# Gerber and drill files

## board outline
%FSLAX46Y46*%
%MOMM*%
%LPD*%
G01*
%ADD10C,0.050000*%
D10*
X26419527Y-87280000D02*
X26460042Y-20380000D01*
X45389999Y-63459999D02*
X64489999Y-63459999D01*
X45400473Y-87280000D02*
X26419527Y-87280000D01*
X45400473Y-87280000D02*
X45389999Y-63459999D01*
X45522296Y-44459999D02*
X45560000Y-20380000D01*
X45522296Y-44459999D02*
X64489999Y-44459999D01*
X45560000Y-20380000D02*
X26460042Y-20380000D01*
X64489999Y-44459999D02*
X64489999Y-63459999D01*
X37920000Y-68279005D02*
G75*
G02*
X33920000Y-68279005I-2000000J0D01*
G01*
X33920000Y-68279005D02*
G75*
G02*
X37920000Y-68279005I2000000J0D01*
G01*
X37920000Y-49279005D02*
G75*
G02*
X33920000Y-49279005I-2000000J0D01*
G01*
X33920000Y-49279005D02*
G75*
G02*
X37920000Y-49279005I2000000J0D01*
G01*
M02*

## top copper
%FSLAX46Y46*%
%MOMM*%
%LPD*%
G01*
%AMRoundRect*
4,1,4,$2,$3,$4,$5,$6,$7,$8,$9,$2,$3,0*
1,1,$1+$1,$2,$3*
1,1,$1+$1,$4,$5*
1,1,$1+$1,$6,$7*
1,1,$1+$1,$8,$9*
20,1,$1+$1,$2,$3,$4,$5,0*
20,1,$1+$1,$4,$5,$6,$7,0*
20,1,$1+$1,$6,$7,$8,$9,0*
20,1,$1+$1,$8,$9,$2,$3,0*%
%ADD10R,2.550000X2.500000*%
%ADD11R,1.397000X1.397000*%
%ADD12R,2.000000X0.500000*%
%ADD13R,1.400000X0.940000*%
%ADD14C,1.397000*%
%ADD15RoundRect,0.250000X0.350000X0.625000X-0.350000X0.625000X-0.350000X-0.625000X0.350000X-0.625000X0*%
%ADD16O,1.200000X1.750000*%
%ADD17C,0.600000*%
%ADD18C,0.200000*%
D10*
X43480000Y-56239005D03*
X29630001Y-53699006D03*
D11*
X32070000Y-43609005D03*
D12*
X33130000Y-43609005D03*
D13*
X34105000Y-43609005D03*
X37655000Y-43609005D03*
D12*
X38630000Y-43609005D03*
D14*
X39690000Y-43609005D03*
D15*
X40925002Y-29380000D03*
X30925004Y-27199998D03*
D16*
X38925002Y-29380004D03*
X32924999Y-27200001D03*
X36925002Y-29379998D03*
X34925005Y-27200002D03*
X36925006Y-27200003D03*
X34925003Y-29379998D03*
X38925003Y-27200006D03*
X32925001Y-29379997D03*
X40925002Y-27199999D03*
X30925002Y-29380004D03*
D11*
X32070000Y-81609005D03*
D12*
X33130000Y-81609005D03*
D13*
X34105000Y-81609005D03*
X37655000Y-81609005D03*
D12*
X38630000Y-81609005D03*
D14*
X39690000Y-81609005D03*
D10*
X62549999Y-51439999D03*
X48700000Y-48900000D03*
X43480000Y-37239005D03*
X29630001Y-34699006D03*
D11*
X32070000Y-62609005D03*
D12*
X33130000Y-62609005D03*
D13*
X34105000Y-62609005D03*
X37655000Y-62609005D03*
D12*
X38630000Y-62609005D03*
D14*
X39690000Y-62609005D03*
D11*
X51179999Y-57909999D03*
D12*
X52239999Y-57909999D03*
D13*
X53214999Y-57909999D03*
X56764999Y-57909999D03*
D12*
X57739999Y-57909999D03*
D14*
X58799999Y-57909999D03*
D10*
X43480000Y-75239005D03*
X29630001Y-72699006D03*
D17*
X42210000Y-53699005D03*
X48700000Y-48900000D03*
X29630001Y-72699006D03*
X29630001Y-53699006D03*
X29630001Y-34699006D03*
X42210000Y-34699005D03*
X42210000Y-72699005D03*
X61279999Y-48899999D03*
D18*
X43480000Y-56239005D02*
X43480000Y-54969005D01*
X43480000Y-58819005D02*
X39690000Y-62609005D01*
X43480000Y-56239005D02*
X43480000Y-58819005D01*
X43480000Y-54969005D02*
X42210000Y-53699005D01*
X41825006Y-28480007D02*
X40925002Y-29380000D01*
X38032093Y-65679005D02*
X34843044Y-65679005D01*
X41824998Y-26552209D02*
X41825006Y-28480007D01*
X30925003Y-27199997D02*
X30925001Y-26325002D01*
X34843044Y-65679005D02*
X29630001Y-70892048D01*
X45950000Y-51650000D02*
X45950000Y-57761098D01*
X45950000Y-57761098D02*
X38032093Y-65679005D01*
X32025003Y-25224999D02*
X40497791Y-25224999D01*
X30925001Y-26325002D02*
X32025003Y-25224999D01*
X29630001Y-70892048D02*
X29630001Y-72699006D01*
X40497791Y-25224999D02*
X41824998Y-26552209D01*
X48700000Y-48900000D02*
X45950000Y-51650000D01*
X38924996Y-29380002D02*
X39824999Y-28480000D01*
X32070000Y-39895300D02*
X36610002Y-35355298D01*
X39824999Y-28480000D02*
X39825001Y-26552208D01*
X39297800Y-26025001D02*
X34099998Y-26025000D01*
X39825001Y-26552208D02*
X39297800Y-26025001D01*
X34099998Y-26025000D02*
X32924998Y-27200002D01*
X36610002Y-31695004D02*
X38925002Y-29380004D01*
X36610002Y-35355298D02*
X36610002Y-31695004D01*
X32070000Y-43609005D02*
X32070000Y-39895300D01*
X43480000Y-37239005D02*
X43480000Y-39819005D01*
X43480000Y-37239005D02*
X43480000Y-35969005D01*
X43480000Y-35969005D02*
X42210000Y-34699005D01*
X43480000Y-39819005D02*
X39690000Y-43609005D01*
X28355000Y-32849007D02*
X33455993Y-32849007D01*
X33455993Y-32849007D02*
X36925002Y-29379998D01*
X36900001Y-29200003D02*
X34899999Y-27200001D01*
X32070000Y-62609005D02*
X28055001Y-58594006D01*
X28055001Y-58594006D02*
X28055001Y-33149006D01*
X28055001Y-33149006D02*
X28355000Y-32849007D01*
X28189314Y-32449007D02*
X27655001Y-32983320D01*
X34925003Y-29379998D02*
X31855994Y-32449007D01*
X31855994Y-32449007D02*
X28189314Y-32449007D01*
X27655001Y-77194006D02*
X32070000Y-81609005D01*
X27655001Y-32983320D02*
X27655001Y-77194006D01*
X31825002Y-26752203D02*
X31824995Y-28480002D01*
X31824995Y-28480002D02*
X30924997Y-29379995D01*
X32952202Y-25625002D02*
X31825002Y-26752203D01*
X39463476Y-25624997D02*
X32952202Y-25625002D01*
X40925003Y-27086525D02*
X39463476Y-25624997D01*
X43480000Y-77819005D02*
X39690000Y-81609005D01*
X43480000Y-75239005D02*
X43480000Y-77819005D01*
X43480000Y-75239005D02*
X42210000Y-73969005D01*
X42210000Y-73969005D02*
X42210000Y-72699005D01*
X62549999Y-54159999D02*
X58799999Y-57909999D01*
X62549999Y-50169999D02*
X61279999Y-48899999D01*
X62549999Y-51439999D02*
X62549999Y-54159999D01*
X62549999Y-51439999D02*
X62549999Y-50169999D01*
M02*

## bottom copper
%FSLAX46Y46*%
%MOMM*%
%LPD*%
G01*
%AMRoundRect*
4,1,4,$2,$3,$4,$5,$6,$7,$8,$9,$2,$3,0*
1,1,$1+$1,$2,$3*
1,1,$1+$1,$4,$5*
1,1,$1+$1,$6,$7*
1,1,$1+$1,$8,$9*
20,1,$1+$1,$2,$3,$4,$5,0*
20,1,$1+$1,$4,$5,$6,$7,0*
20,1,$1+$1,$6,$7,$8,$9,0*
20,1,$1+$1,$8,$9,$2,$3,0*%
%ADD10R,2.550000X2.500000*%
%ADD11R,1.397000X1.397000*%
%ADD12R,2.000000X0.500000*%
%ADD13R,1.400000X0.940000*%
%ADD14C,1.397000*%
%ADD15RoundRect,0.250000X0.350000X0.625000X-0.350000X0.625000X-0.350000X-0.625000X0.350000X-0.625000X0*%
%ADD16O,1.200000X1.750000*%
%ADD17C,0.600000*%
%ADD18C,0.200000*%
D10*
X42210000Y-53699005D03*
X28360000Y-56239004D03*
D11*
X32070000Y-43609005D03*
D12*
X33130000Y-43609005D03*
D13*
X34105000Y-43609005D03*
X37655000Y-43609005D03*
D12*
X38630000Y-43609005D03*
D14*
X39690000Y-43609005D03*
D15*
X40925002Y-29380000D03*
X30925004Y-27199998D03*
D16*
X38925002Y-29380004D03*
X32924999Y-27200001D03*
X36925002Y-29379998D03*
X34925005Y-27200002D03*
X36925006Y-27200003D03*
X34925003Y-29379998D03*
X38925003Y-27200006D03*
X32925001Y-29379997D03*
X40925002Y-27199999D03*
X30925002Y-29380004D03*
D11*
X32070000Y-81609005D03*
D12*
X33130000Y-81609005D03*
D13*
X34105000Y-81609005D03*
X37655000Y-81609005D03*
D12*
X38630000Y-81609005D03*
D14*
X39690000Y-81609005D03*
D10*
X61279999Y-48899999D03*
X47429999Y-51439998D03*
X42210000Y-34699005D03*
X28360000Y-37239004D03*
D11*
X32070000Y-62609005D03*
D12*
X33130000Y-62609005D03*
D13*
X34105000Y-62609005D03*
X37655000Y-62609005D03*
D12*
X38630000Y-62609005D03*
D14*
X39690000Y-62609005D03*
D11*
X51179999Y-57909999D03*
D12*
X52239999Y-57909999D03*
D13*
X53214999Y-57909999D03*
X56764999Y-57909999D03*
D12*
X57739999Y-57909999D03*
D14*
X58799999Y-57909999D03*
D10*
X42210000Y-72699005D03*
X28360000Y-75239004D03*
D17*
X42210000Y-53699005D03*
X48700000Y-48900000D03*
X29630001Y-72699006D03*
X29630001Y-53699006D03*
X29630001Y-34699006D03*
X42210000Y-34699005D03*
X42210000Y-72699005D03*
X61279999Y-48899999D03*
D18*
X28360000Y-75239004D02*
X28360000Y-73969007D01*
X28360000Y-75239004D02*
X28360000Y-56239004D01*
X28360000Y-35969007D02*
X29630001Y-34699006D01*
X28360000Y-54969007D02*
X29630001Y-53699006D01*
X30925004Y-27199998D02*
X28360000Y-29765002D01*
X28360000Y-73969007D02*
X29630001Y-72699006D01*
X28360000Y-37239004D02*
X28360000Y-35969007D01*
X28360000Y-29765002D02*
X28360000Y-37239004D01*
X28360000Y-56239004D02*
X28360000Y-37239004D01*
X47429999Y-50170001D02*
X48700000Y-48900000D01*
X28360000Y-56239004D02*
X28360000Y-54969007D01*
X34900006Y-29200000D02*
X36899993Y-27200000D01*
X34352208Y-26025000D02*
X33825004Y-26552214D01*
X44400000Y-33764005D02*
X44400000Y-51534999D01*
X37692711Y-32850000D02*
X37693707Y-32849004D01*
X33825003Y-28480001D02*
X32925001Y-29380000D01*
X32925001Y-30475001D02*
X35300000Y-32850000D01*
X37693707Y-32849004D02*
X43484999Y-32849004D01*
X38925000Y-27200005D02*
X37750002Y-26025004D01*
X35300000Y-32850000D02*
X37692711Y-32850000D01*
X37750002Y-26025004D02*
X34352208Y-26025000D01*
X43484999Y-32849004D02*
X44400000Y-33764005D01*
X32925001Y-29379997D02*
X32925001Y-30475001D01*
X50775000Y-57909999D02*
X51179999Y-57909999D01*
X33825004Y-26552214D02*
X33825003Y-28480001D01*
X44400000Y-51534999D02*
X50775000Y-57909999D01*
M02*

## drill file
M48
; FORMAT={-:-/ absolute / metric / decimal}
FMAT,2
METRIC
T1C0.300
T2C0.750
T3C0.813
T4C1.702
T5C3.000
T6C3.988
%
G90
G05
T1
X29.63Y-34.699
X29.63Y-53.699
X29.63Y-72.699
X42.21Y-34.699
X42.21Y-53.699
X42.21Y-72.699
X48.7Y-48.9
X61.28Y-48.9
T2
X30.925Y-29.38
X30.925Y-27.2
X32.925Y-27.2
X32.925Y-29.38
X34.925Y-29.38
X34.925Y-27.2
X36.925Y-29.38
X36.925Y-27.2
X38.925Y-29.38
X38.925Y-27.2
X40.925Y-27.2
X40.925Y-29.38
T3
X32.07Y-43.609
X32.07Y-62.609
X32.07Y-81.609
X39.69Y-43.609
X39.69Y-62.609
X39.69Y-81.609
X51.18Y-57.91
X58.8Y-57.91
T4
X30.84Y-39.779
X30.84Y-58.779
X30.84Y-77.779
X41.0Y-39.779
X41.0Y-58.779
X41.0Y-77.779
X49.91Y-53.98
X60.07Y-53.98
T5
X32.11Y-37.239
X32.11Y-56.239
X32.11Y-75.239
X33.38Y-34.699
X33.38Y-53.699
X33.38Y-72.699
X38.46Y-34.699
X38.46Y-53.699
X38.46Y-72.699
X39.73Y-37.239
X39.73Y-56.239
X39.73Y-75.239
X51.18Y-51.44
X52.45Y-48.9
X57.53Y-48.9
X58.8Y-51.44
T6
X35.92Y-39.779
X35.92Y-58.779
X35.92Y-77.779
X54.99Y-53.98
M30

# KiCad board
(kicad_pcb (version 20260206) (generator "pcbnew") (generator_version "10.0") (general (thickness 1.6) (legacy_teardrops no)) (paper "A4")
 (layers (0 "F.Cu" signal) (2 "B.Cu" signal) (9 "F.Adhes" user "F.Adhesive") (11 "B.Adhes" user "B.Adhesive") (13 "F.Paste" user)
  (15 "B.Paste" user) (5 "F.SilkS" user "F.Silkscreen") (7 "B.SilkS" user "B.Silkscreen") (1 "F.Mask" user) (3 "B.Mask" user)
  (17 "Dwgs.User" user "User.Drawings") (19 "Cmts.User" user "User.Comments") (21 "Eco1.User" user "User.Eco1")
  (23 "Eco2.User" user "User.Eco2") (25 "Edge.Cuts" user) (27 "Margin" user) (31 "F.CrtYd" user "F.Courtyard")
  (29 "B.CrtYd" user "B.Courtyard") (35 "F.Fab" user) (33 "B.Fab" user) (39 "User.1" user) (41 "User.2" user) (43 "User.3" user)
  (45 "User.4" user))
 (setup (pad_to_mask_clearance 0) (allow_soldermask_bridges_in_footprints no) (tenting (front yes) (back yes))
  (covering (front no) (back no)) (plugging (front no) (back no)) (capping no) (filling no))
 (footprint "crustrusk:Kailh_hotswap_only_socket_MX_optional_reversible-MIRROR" (layer "F.Cu") (at 35.92 58.779005)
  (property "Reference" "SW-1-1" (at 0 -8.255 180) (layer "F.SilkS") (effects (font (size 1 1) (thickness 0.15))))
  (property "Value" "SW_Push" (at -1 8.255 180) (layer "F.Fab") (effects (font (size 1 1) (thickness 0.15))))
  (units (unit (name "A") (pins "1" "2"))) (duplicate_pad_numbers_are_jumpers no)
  (pad "" np_thru_hole circle (at -5.08 0) (size 1.7018 1.7018) (drill 1.7018) (layers "*.Cu" "*.Mask"))
  (pad "" np_thru_hole circle (at -3.81 -2.54 180) (size 3 3) (drill 3) (layers "*.Cu" "*.Mask"))
  (pad "" np_thru_hole circle (at -2.54 -5.079998) (size 3 3) (drill 3) (layers "*.Cu" "*.Mask"))
  (pad "" np_thru_hole circle (at 0 0) (size 3.9878 3.9878) (drill 3.9878) (layers "*.Cu" "*.Mask"))
  (pad "" np_thru_hole circle (at 2.540002 -5.080001 180) (size 3 3) (drill 3) (layers "*.Cu" "*.Mask"))
  (pad "" np_thru_hole circle (at 3.81 -2.54) (size 3 3) (drill 3) (layers "*.Cu" "*.Mask"))
  (pad "" np_thru_hole circle (at 5.08 0) (size 1.7018 1.7018) (drill 1.7018) (layers "*.Cu" "*.Mask"))
  (pad "1" smd rect (at 6.29 -5.08 180) (size 2.55 2.5) (layers "B.Cu" "B.Mask" "B.Paste") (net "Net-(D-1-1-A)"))
  (pad "1" smd rect (at 7.56 -2.54) (size 2.55 2.5) (layers "F.Cu" "F.Mask" "F.Paste") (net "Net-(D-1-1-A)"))
  (pad "2" smd rect (at -7.56 -2.540001 180) (size 2.55 2.5) (layers "B.Cu" "B.Mask" "B.Paste") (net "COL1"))
  (pad "2" smd rect (at -6.289999 -5.079999) (size 2.55 2.5) (layers "F.Cu" "F.Mask" "F.Paste") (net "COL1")))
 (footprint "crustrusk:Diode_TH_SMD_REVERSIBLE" (layer "F.Cu") (at 35.88 43.609005)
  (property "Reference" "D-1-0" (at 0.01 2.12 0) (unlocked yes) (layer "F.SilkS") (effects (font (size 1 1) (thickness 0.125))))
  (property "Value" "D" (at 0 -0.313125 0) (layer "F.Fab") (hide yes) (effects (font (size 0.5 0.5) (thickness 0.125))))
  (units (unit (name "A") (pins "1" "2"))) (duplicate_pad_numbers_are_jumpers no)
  (pad "1" thru_hole rect (at -3.81 0) (size 1.397 1.397) (drill 0.8128) (layers "*.Cu" "*.Mask") (remove_unused_layers no) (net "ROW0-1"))
  (pad "1" smd rect (at -2.75 0 180) (size 2 0.5) (layers "F.Cu") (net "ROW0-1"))
  (pad "1" smd rect (at -2.75 0) (size 2 0.5) (layers "B.Cu") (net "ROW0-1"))
  (pad "1" smd rect (at -1.775 0 180) (size 1.4 0.94) (layers "F.Cu" "F.Mask" "F.Paste") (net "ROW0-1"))
  (pad "1" smd rect (at -1.775 0) (size 1.4 0.94) (layers "B.Cu" "B.Mask" "B.Paste") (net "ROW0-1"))
  (pad "2" smd rect (at 1.775 0 180) (size 1.4 0.94) (layers "F.Cu" "F.Mask" "F.Paste") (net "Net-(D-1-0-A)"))
  (pad "2" smd rect (at 1.775 0) (size 1.4 0.94) (layers "B.Cu" "B.Mask" "B.Paste") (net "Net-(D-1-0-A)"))
  (pad "2" smd rect (at 2.75 0 180) (size 2 0.5) (layers "F.Cu") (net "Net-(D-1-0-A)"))
  (pad "2" smd rect (at 2.75 0) (size 2 0.5) (layers "B.Cu") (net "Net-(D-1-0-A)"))
  (pad "2" thru_hole circle (at 3.81 0) (size 1.397 1.397) (drill 0.8128) (layers "*.Cu" "*.Mask") (remove_unused_layers no)
   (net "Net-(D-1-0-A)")))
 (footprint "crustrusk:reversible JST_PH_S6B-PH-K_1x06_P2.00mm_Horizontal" (layer "F.Cu") (at 40.925002 29.38 180)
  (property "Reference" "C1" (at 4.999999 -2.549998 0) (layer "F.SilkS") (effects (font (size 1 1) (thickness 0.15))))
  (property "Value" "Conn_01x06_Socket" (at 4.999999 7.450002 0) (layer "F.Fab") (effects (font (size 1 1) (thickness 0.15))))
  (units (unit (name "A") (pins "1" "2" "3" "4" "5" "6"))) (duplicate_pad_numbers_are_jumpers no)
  (pad "1" thru_hole roundrect (at 0 0 180) (size 1.2 1.75) (drill 0.75) (layers "*.Cu" "*.Mask") (remove_unused_layers no)
   (roundrect_rratio 0.208333) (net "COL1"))
  (pad "1" thru_hole roundrect (at 9.999998 2.180002 180) (size 1.2 1.75) (drill 0.75) (layers "*.Cu" "*.Mask") (remove_unused_layers no)
   (roundrect_rratio 0.208333) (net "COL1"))
  (pad "2" thru_hole oval (at 2 -0.000004 180) (size 1.2 1.75) (drill 0.75) (layers "*.Cu" "*.Mask") (remove_unused_layers no)
   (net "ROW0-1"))
  (pad "2" thru_hole oval (at 8.000003 2.179999 180) (size 1.2 1.75) (drill 0.75) (layers "*.Cu" "*.Mask") (remove_unused_layers no)
   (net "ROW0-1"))
  (pad "3" thru_hole oval (at 4 0.000002 180) (size 1.2 1.75) (drill 0.75) (layers "*.Cu" "*.Mask") (remove_unused_layers no) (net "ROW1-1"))
  (pad "3" thru_hole oval (at 5.999997 2.179998 180) (size 1.2 1.75) (drill 0.75) (layers "*.Cu" "*.Mask") (remove_unused_layers no)
   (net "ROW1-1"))
  (pad "4" thru_hole oval (at 3.999996 2.179997 180) (size 1.2 1.75) (drill 0.75) (layers "*.Cu" "*.Mask") (remove_unused_layers no)
   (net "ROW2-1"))
  (pad "4" thru_hole oval (at 5.999999 0.000002 180) (size 1.2 1.75) (drill 0.75) (layers "*.Cu" "*.Mask") (remove_unused_layers no)
   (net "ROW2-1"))
  (pad "5" thru_hole oval (at 1.999999 2.179994 180) (size 1.2 1.75) (drill 0.75) (layers "*.Cu" "*.Mask") (remove_unused_layers no)
   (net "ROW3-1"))
  (pad "5" thru_hole oval (at 8.000001 0.000003 180) (size 1.2 1.75) (drill 0.75) (layers "*.Cu" "*.Mask") (remove_unused_layers no)
   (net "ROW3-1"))
  (pad "6" thru_hole oval (at 0 2.180001 180) (size 1.2 1.75) (drill 0.75) (layers "*.Cu" "*.Mask") (remove_unused_layers no) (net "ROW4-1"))
  (pad "6" thru_hole oval (at 10 -0.000004 180) (size 1.2 1.75) (drill 0.75) (layers "*.Cu" "*.Mask") (remove_unused_layers no)
   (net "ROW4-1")))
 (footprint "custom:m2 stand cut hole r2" (layer "F.Cu") (at 35.92 68.279005)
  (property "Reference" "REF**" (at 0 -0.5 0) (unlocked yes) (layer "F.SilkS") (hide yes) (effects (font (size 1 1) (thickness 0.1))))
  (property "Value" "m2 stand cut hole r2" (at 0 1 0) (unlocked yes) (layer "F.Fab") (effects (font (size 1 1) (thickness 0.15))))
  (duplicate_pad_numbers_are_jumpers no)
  (fp_circle (center 0 0) (end 2 0) (stroke (width 0.05) (type default)) (fill no) (layer "Edge.Cuts")))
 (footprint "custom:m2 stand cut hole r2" (layer "F.Cu") (at 35.92 49.279005)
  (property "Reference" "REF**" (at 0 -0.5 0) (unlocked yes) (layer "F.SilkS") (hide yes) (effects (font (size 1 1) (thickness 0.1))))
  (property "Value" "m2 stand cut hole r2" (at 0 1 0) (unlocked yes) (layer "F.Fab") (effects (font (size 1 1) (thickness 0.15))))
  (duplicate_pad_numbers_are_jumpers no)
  (fp_circle (center 0 0) (end 2 0) (stroke (width 0.05) (type default)) (fill no) (layer "Edge.Cuts")))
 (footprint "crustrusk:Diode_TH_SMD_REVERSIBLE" (layer "F.Cu") (at 35.88 81.609005)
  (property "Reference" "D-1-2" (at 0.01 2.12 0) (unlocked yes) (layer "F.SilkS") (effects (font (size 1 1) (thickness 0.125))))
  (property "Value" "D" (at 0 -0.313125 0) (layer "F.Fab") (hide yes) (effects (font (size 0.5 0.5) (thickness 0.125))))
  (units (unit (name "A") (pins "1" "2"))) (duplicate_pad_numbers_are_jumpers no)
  (pad "1" thru_hole rect (at -3.81 0) (size 1.397 1.397) (drill 0.8128) (layers "*.Cu" "*.Mask") (remove_unused_layers no) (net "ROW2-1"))
  (pad "1" smd rect (at -2.75 0 180) (size 2 0.5) (layers "F.Cu") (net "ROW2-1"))
  (pad "1" smd rect (at -2.75 0) (size 2 0.5) (layers "B.Cu") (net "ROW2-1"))
  (pad "1" smd rect (at -1.775 0 180) (size 1.4 0.94) (layers "F.Cu" "F.Mask" "F.Paste") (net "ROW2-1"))
  (pad "1" smd rect (at -1.775 0) (size 1.4 0.94) (layers "B.Cu" "B.Mask" "B.Paste") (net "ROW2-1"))
  (pad "2" smd rect (at 1.775 0 180) (size 1.4 0.94) (layers "F.Cu" "F.Mask" "F.Paste") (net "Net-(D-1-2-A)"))
  (pad "2" smd rect (at 1.775 0) (size 1.4 0.94) (layers "B.Cu" "B.Mask" "B.Paste") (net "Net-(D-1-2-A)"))
  (pad "2" smd rect (at 2.75 0 180) (size 2 0.5) (layers "F.Cu") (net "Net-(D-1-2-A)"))
  (pad "2" smd rect (at 2.75 0) (size 2 0.5) (layers "B.Cu") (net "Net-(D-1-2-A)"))
  (pad "2" thru_hole circle (at 3.81 0) (size 1.397 1.397) (drill 0.8128) (layers "*.Cu" "*.Mask") (remove_unused_layers no)
   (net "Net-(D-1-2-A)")))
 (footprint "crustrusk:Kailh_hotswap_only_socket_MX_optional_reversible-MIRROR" (layer "F.Cu") (at 54.989999 53.979999)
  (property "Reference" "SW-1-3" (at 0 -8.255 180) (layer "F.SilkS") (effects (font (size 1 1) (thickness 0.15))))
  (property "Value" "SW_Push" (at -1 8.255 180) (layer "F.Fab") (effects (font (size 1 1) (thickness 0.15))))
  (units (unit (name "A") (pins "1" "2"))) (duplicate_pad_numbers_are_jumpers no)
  (pad "" np_thru_hole circle (at -5.08 0) (size 1.7018 1.7018) (drill 1.7018) (layers "*.Cu" "*.Mask"))
  (pad "" np_thru_hole circle (at -3.81 -2.54 180) (size 3 3) (drill 3) (layers "*.Cu" "*.Mask"))
  (pad "" np_thru_hole circle (at -2.54 -5.079998) (size 3 3) (drill 3) (layers "*.Cu" "*.Mask"))
  (pad "" np_thru_hole circle (at 0 0) (size 3.9878 3.9878) (drill 3.9878) (layers "*.Cu" "*.Mask"))
  (pad "" np_thru_hole circle (at 2.540002 -5.080001 180) (size 3 3) (drill 3) (layers "*.Cu" "*.Mask"))
  (pad "" np_thru_hole circle (at 3.81 -2.54) (size 3 3) (drill 3) (layers "*.Cu" "*.Mask"))
  (pad "" np_thru_hole circle (at 5.08 0) (size 1.7018 1.7018) (drill 1.7018) (layers "*.Cu" "*.Mask"))
  (pad "1" smd rect (at 6.29 -5.08 180) (size 2.55 2.5) (layers "B.Cu" "B.Mask" "B.Paste") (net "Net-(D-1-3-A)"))
  (pad "1" smd rect (at 7.56 -2.54) (size 2.55 2.5) (layers "F.Cu" "F.Mask" "F.Paste") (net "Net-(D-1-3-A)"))
  (pad "2" smd rect (at -7.56 -2.540001 180) (size 2.55 2.5) (layers "B.Cu" "B.Mask" "B.Paste") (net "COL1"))
  (pad "2" smd rect (at -6.289999 -5.079999) (size 2.55 2.5) (layers "F.Cu" "F.Mask" "F.Paste") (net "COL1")))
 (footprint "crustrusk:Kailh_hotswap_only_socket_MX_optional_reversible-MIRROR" (layer "F.Cu") (at 35.92 39.779005)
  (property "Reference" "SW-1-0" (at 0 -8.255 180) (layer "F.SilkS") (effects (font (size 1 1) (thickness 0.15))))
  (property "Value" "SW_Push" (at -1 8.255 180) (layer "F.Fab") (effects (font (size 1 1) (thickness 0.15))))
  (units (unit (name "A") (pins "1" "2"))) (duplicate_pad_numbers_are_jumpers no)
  (pad "" np_thru_hole circle (at -5.08 0) (size 1.7018 1.7018) (drill 1.7018) (layers "*.Cu" "*.Mask"))
  (pad "" np_thru_hole circle (at -3.81 -2.54 180) (size 3 3) (drill 3) (layers "*.Cu" "*.Mask"))
  (pad "" np_thru_hole circle (at -2.54 -5.079998) (size 3 3) (drill 3) (layers "*.Cu" "*.Mask"))
  (pad "" np_thru_hole circle (at 0 0) (size 3.9878 3.9878) (drill 3.9878) (layers "*.Cu" "*.Mask"))
  (pad "" np_thru_hole circle (at 2.540002 -5.080001 180) (size 3 3) (drill 3) (layers "*.Cu" "*.Mask"))
  (pad "" np_thru_hole circle (at 3.81 -2.54) (size 3 3) (drill 3) (layers "*.Cu" "*.Mask"))
  (pad "" np_thru_hole circle (at 5.08 0) (size 1.7018 1.7018) (drill 1.7018) (layers "*.Cu" "*.Mask"))
  (pad "1" smd rect (at 6.29 -5.08 180) (size 2.55 2.5) (layers "B.Cu" "B.Mask" "B.Paste") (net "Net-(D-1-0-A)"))
  (pad "1" smd rect (at 7.56 -2.54) (size 2.55 2.5) (layers "F.Cu" "F.Mask" "F.Paste") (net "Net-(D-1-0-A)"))
  (pad "2" smd rect (at -7.56 -2.540001 180) (size 2.55 2.5) (layers "B.Cu" "B.Mask" "B.Paste") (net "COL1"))
  (pad "2" smd rect (at -6.289999 -5.079999) (size 2.55 2.5) (layers "F.Cu" "F.Mask" "F.Paste") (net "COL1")))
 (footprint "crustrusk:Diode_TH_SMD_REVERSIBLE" (layer "F.Cu") (at 35.88 62.609005)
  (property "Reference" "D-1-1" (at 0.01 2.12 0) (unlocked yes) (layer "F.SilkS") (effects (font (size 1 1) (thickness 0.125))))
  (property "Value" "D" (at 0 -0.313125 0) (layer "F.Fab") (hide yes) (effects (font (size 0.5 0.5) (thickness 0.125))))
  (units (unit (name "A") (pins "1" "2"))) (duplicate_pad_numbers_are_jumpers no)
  (pad "1" thru_hole rect (at -3.81 0) (size 1.397 1.397) (drill 0.8128) (layers "*.Cu" "*.Mask") (remove_unused_layers no) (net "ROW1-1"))
  (pad "1" smd rect (at -2.75 0 180) (size 2 0.5) (layers "F.Cu") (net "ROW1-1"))
  (pad "1" smd rect (at -2.75 0) (size 2 0.5) (layers "B.Cu") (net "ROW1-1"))
  (pad "1" smd rect (at -1.775 0 180) (size 1.4 0.94) (layers "F.Cu" "F.Mask" "F.Paste") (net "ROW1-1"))
  (pad "1" smd rect (at -1.775 0) (size 1.4 0.94) (layers "B.Cu" "B.Mask" "B.Paste") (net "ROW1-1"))
  (pad "2" smd rect (at 1.775 0 180) (size 1.4 0.94) (layers "F.Cu" "F.Mask" "F.Paste") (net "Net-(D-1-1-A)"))
  (pad "2" smd rect (at 1.775 0) (size 1.4 0.94) (layers "B.Cu" "B.Mask" "B.Paste") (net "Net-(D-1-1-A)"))
  (pad "2" smd rect (at 2.75 0 180) (size 2 0.5) (layers "F.Cu") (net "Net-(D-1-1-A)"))
  (pad "2" smd rect (at 2.75 0) (size 2 0.5) (layers "B.Cu") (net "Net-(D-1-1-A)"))
  (pad "2" thru_hole circle (at 3.81 0) (size 1.397 1.397) (drill 0.8128) (layers "*.Cu" "*.Mask") (remove_unused_layers no)
   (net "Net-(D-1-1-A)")))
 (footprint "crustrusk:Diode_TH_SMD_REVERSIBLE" (layer "F.Cu") (at 54.989999 57.909999)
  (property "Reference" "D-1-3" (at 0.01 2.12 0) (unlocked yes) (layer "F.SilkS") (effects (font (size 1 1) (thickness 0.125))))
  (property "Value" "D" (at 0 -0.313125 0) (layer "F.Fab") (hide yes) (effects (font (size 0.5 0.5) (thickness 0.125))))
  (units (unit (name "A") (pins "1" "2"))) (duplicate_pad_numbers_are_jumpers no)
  (pad "1" thru_hole rect (at -3.81 0) (size 1.397 1.397) (drill 0.8128) (layers "*.Cu" "*.Mask") (remove_unused_layers no) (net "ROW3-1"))
  (pad "1" smd rect (at -2.75 0 180) (size 2 0.5) (layers "F.Cu") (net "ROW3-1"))
  (pad "1" smd rect (at -2.75 0) (size 2 0.5) (layers "B.Cu") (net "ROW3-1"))
  (pad "1" smd rect (at -1.775 0 180) (size 1.4 0.94) (layers "F.Cu" "F.Mask" "F.Paste") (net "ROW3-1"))
  (pad "1" smd rect (at -1.775 0) (size 1.4 0.94) (layers "B.Cu" "B.Mask" "B.Paste") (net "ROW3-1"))
  (pad "2" smd rect (at 1.775 0 180) (size 1.4 0.94) (layers "F.Cu" "F.Mask" "F.Paste") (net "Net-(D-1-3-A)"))
  (pad "2" smd rect (at 1.775 0) (size 1.4 0.94) (layers "B.Cu" "B.Mask" "B.Paste") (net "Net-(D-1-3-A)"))
  (pad "2" smd rect (at 2.75 0 180) (size 2 0.5) (layers "F.Cu") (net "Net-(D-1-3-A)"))
  (pad "2" smd rect (at 2.75 0) (size 2 0.5) (layers "B.Cu") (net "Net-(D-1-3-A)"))
  (pad "2" thru_hole circle (at 3.81 0) (size 1.397 1.397) (drill 0.8128) (layers "*.Cu" "*.Mask") (remove_unused_layers no)
   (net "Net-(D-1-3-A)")))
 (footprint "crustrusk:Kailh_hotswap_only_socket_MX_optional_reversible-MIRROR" (layer "F.Cu") (at 35.92 77.779005)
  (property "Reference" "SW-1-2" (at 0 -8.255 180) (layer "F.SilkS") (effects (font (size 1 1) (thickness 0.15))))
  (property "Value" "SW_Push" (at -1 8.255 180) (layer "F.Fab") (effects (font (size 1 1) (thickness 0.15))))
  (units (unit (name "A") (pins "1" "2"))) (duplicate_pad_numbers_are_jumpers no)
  (pad "" np_thru_hole circle (at -5.08 0) (size 1.7018 1.7018) (drill 1.7018) (layers "*.Cu" "*.Mask"))
  (pad "" np_thru_hole circle (at -3.81 -2.54 180) (size 3 3) (drill 3) (layers "*.Cu" "*.Mask"))
  (pad "" np_thru_hole circle (at -2.54 -5.079998) (size 3 3) (drill 3) (layers "*.Cu" "*.Mask"))
  (pad "" np_thru_hole circle (at 0 0) (size 3.9878 3.9878) (drill 3.9878) (layers "*.Cu" "*.Mask"))
  (pad "" np_thru_hole circle (at 2.540002 -5.080001 180) (size 3 3) (drill 3) (layers "*.Cu" "*.Mask"))
  (pad "" np_thru_hole circle (at 3.81 -2.54) (size 3 3) (drill 3) (layers "*.Cu" "*.Mask"))
  (pad "" np_thru_hole circle (at 5.08 0) (size 1.7018 1.7018) (drill 1.7018) (layers "*.Cu" "*.Mask"))
  (pad "1" smd rect (at 6.29 -5.08 180) (size 2.55 2.5) (layers "B.Cu" "B.Mask" "B.Paste") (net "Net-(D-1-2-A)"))
  (pad "1" smd rect (at 7.56 -2.54) (size 2.55 2.5) (layers "F.Cu" "F.Mask" "F.Paste") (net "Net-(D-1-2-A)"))
  (pad "2" smd rect (at -7.56 -2.540001 180) (size 2.55 2.5) (layers "B.Cu" "B.Mask" "B.Paste") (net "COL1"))
  (pad "2" smd rect (at -6.289999 -5.079999) (size 2.55 2.5) (layers "F.Cu" "F.Mask" "F.Paste") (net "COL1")))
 (gr_line (start 26.419527 87.28) (end 26.460042 20.38) (stroke (width 0.05) (type default)) (layer "Edge.Cuts"))
 (gr_line (start 45.389999 63.459999) (end 64.489999 63.459999) (stroke (width 0.05) (type default)) (layer "Edge.Cuts"))
 (gr_line (start 45.400473 87.28) (end 26.419527 87.28) (stroke (width 0.05) (type default)) (layer "Edge.Cuts"))
 (gr_line (start 45.400473 87.28) (end 45.389999 63.459999) (stroke (width 0.05) (type default)) (layer "Edge.Cuts"))
 (gr_line (start 45.522296 44.459999) (end 45.56 20.38) (stroke (width 0.05) (type default)) (layer "Edge.Cuts"))
 (gr_line (start 45.522296 44.459999) (end 64.489999 44.459999) (stroke (width 0.05) (type default)) (layer "Edge.Cuts"))
 (gr_line (start 45.56 20.38) (end 26.460042 20.38) (stroke (width 0.05) (type default)) (layer "Edge.Cuts"))
 (gr_line (start 64.489999 44.459999) (end 64.489999 63.459999) (stroke (width 0.05) (type default)) (layer "Edge.Cuts"))
 (segment (start 43.48 56.239005) (end 43.48 54.969005) (width 0.2) (layer "F.Cu") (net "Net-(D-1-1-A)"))
 (segment (start 43.48 58.819005) (end 39.69 62.609005) (width 0.2) (layer "F.Cu") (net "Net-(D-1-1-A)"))
 (segment (start 43.48 56.239005) (end 43.48 58.819005) (width 0.2) (layer "F.Cu") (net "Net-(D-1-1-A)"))
 (segment (start 43.48 54.969005) (end 42.21 53.699005) (width 0.2) (layer "F.Cu") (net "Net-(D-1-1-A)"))
 (via (at 42.21 53.699005) (size 0.6) (drill 0.3) (layers "F.Cu" "B.Cu") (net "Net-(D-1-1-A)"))
 (segment (start 41.825006 28.480007) (end 40.925002 29.38) (width 0.2) (layer "F.Cu") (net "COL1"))
 (segment (start 38.032093 65.679005) (end 34.843044 65.679005) (width 0.2) (layer "F.Cu") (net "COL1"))
 (segment (start 41.824998 26.552209) (end 41.825006 28.480007) (width 0.2) (layer "F.Cu") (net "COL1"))
 (segment (start 30.925003 27.199997) (end 30.925001 26.325002) (width 0.2) (layer "F.Cu") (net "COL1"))
 (segment (start 34.843044 65.679005) (end 29.630001 70.892048) (width 0.2) (layer "F.Cu") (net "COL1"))
 (segment (start 45.95 51.65) (end 45.95 57.761098) (width 0.2) (layer "F.Cu") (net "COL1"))
 (segment (start 45.95 57.761098) (end 38.032093 65.679005) (width 0.2) (layer "F.Cu") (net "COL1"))
 (segment (start 32.025003 25.224999) (end 40.497791 25.224999) (width 0.2) (layer "F.Cu") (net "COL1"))
 (segment (start 30.925001 26.325002) (end 32.025003 25.224999) (width 0.2) (layer "F.Cu") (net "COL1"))
 (segment (start 29.630001 70.892048) (end 29.630001 72.699006) (width 0.2) (layer "F.Cu") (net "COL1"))
 (segment (start 40.497791 25.224999) (end 41.824998 26.552209) (width 0.2) (layer "F.Cu") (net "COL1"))
 (segment (start 48.7 48.9) (end 45.95 51.65) (width 0.2) (layer "F.Cu") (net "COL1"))
 (via (at 48.7 48.9) (size 0.6) (drill 0.3) (layers "F.Cu" "B.Cu") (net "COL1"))
 (via (at 29.630001 72.699006) (size 0.6) (drill 0.3) (layers "F.Cu" "B.Cu") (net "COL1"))
 (via (at 29.630001 53.699006) (size 0.6) (drill 0.3) (layers "F.Cu" "B.Cu") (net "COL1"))
 (via (at 29.630001 34.699006) (size 0.6) (drill 0.3) (layers "F.Cu" "B.Cu") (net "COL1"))
 (segment (start 28.36 75.239004) (end 28.36 73.969007) (width 0.2) (layer "B.Cu") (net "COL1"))
 (segment (start 28.36 75.239004) (end 28.36 56.239004) (width 0.2) (layer "B.Cu") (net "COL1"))
 (segment (start 28.36 35.969007) (end 29.630001 34.699006) (width 0.2) (layer "B.Cu") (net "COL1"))
 (segment (start 28.36 54.969007) (end 29.630001 53.699006) (width 0.2) (layer "B.Cu") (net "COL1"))
 (segment (start 30.925004 27.199998) (end 28.36 29.765002) (width 0.2) (layer "B.Cu") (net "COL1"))
 (segment (start 28.36 73.969007) (end 29.630001 72.699006) (width 0.2) (layer "B.Cu") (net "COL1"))
 (segment (start 28.36 37.239004) (end 28.36 35.969007) (width 0.2) (layer "B.Cu") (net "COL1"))
 (segment (start 28.36 29.765002) (end 28.36 37.239004) (width 0.2) (layer "B.Cu") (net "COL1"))
 (segment (start 28.36 56.239004) (end 28.36 37.239004) (width 0.2) (layer "B.Cu") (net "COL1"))
 (segment (start 47.429999 50.170001) (end 48.7 48.9) (width 0.2) (layer "B.Cu") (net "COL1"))
 (segment (start 28.36 56.239004) (end 28.36 54.969007) (width 0.2) (layer "B.Cu") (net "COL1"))
 (segment (start 38.924996 29.380002) (end 39.824999 28.48) (width 0.2) (layer "F.Cu") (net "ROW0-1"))
 (segment (start 32.07 39.8953) (end 36.610002 35.355298) (width 0.2) (layer "F.Cu") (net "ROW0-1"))
 (segment (start 39.824999 28.48) (end 39.825001 26.552208) (width 0.2) (layer "F.Cu") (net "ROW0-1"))
 (segment (start 39.2978 26.025001) (end 34.099998 26.025) (width 0.2) (layer "F.Cu") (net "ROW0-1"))
 (segment (start 39.825001 26.552208) (end 39.2978 26.025001) (width 0.2) (layer "F.Cu") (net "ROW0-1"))
 (segment (start 34.099998 26.025) (end 32.924998 27.200002) (width 0.2) (layer "F.Cu") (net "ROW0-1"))
 (segment (start 36.610002 31.695004) (end 38.925002 29.380004) (width 0.2) (layer "F.Cu") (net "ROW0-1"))
 (segment (start 36.610002 35.355298) (end 36.610002 31.695004) (width 0.2) (layer "F.Cu") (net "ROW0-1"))
 (segment (start 32.07 43.609005) (end 32.07 39.8953) (width 0.2) (layer "F.Cu") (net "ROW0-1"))
 (segment (start 43.48 37.239005) (end 43.48 39.819005) (width 0.2) (layer "F.Cu") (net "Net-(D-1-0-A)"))
 (segment (start 43.48 37.239005) (end 43.48 35.969005) (width 0.2) (layer "F.Cu") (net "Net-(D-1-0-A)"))
 (segment (start 43.48 35.969005) (end 42.21 34.699005) (width 0.2) (layer "F.Cu") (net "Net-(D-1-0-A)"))
 (segment (start 43.48 39.819005) (end 39.69 43.609005) (width 0.2) (layer "F.Cu") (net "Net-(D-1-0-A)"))
 (via (at 42.21 34.699005) (size 0.6) (drill 0.3) (layers "F.Cu" "B.Cu") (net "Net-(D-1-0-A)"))
 (segment (start 28.355 32.849007) (end 33.455993 32.849007) (width 0.2) (layer "F.Cu") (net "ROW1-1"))
 (segment (start 33.455993 32.849007) (end 36.925002 29.379998) (width 0.2) (layer "F.Cu") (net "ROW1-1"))
 (segment (start 36.900001 29.200003) (end 34.899999 27.200001) (width 0.2) (layer "F.Cu") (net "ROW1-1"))
 (segment (start 32.07 62.609005) (end 28.055001 58.594006) (width 0.2) (layer "F.Cu") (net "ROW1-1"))
 (segment (start 28.055001 58.594006) (end 28.055001 33.149006) (width 0.2) (layer "F.Cu") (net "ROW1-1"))
 (segment (start 28.055001 33.149006) (end 28.355 32.849007) (width 0.2) (layer "F.Cu") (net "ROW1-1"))
 (segment (start 28.189314 32.449007) (end 27.655001 32.98332) (width 0.2) (layer "F.Cu") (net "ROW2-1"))
 (segment (start 34.925003 29.379998) (end 31.855994 32.449007) (width 0.2) (layer "F.Cu") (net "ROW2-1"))
 (segment (start 31.855994 32.449007) (end 28.189314 32.449007) (width 0.2) (layer "F.Cu") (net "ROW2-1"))
 (segment (start 27.655001 77.194006) (end 32.07 81.609005) (width 0.2) (layer "F.Cu") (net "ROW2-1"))
 (segment (start 27.655001 32.98332) (end 27.655001 77.194006) (width 0.2) (layer "F.Cu") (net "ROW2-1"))
 (segment (start 34.900006 29.2) (end 36.899993 27.2) (width 0.2) (layer "B.Cu") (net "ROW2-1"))
 (segment (start 34.352208 26.025) (end 33.825004 26.552214) (width 0.2) (layer "B.Cu") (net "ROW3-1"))
 (segment (start 44.4 33.764005) (end 44.4 51.534999) (width 0.2) (layer "B.Cu") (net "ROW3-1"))
 (segment (start 37.692711 32.85) (end 37.693707 32.849004) (width 0.2) (layer "B.Cu") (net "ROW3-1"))
 (segment (start 33.825003 28.480001) (end 32.925001 29.38) (width 0.2) (layer "B.Cu") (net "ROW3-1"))
 (segment (start 32.925001 30.475001) (end 35.3 32.85) (width 0.2) (layer "B.Cu") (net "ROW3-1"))
 (segment (start 37.693707 32.849004) (end 43.484999 32.849004) (width 0.2) (layer "B.Cu") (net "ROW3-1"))
 (segment (start 38.925 27.200005) (end 37.750002 26.025004) (width 0.2) (layer "B.Cu") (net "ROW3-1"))
 (segment (start 35.3 32.85) (end 37.692711 32.85) (width 0.2) (layer "B.Cu") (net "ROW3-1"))
 (segment (start 37.750002 26.025004) (end 34.352208 26.025) (width 0.2) (layer "B.Cu") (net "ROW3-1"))
 (segment (start 43.484999 32.849004) (end 44.4 33.764005) (width 0.2) (layer "B.Cu") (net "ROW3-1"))
 (segment (start 32.925001 29.379997) (end 32.925001 30.475001) (width 0.2) (layer "B.Cu") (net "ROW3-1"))
 (segment (start 50.775 57.909999) (end 51.179999 57.909999) (width 0.2) (layer "B.Cu") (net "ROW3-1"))
 (segment (start 33.825004 26.552214) (end 33.825003 28.480001) (width 0.2) (layer "B.Cu") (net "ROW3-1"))
 (segment (start 44.4 51.534999) (end 50.775 57.909999) (width 0.2) (layer "B.Cu") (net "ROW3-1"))
 (segment (start 31.825002 26.752203) (end 31.824995 28.480002) (width 0.2) (layer "F.Cu") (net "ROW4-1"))
 (segment (start 31.824995 28.480002) (end 30.924997 29.379995) (width 0.2) (layer "F.Cu") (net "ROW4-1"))
 (segment (start 32.952202 25.625002) (end 31.825002 26.752203) (width 0.2) (layer "F.Cu") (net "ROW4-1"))
 (segment (start 39.463476 25.624997) (end 32.952202 25.625002) (width 0.2) (layer "F.Cu") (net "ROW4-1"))
 (segment (start 40.925003 27.086525) (end 39.463476 25.624997) (width 0.2) (layer "F.Cu") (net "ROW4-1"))
 (segment (start 43.48 77.819005) (end 39.69 81.609005) (width 0.2) (layer "F.Cu") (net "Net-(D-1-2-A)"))
 (segment (start 43.48 75.239005) (end 43.48 77.819005) (width 0.2) (layer "F.Cu") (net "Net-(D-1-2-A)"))
 (segment (start 43.48 75.239005) (end 42.21 73.969005) (width 0.2) (layer "F.Cu") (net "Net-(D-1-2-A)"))
 (segment (start 42.21 73.969005) (end 42.21 72.699005) (width 0.2) (layer "F.Cu") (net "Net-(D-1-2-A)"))
 (via (at 42.21 72.699005) (size 0.6) (drill 0.3) (layers "F.Cu" "B.Cu") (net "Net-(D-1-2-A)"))
 (segment (start 62.549999 54.159999) (end 58.799999 57.909999) (width 0.2) (layer "F.Cu") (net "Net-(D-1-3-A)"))
 (segment (start 62.549999 50.169999) (end 61.279999 48.899999) (width 0.2) (layer "F.Cu") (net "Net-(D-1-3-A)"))
 (segment (start 62.549999 51.439999) (end 62.549999 54.159999) (width 0.2) (layer "F.Cu") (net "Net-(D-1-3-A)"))
 (segment (start 62.549999 51.439999) (end 62.549999 50.169999) (width 0.2) (layer "F.Cu") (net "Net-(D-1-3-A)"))
 (via (at 61.279999 48.899999) (size 0.6) (drill 0.3) (layers "F.Cu" "B.Cu") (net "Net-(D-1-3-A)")))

